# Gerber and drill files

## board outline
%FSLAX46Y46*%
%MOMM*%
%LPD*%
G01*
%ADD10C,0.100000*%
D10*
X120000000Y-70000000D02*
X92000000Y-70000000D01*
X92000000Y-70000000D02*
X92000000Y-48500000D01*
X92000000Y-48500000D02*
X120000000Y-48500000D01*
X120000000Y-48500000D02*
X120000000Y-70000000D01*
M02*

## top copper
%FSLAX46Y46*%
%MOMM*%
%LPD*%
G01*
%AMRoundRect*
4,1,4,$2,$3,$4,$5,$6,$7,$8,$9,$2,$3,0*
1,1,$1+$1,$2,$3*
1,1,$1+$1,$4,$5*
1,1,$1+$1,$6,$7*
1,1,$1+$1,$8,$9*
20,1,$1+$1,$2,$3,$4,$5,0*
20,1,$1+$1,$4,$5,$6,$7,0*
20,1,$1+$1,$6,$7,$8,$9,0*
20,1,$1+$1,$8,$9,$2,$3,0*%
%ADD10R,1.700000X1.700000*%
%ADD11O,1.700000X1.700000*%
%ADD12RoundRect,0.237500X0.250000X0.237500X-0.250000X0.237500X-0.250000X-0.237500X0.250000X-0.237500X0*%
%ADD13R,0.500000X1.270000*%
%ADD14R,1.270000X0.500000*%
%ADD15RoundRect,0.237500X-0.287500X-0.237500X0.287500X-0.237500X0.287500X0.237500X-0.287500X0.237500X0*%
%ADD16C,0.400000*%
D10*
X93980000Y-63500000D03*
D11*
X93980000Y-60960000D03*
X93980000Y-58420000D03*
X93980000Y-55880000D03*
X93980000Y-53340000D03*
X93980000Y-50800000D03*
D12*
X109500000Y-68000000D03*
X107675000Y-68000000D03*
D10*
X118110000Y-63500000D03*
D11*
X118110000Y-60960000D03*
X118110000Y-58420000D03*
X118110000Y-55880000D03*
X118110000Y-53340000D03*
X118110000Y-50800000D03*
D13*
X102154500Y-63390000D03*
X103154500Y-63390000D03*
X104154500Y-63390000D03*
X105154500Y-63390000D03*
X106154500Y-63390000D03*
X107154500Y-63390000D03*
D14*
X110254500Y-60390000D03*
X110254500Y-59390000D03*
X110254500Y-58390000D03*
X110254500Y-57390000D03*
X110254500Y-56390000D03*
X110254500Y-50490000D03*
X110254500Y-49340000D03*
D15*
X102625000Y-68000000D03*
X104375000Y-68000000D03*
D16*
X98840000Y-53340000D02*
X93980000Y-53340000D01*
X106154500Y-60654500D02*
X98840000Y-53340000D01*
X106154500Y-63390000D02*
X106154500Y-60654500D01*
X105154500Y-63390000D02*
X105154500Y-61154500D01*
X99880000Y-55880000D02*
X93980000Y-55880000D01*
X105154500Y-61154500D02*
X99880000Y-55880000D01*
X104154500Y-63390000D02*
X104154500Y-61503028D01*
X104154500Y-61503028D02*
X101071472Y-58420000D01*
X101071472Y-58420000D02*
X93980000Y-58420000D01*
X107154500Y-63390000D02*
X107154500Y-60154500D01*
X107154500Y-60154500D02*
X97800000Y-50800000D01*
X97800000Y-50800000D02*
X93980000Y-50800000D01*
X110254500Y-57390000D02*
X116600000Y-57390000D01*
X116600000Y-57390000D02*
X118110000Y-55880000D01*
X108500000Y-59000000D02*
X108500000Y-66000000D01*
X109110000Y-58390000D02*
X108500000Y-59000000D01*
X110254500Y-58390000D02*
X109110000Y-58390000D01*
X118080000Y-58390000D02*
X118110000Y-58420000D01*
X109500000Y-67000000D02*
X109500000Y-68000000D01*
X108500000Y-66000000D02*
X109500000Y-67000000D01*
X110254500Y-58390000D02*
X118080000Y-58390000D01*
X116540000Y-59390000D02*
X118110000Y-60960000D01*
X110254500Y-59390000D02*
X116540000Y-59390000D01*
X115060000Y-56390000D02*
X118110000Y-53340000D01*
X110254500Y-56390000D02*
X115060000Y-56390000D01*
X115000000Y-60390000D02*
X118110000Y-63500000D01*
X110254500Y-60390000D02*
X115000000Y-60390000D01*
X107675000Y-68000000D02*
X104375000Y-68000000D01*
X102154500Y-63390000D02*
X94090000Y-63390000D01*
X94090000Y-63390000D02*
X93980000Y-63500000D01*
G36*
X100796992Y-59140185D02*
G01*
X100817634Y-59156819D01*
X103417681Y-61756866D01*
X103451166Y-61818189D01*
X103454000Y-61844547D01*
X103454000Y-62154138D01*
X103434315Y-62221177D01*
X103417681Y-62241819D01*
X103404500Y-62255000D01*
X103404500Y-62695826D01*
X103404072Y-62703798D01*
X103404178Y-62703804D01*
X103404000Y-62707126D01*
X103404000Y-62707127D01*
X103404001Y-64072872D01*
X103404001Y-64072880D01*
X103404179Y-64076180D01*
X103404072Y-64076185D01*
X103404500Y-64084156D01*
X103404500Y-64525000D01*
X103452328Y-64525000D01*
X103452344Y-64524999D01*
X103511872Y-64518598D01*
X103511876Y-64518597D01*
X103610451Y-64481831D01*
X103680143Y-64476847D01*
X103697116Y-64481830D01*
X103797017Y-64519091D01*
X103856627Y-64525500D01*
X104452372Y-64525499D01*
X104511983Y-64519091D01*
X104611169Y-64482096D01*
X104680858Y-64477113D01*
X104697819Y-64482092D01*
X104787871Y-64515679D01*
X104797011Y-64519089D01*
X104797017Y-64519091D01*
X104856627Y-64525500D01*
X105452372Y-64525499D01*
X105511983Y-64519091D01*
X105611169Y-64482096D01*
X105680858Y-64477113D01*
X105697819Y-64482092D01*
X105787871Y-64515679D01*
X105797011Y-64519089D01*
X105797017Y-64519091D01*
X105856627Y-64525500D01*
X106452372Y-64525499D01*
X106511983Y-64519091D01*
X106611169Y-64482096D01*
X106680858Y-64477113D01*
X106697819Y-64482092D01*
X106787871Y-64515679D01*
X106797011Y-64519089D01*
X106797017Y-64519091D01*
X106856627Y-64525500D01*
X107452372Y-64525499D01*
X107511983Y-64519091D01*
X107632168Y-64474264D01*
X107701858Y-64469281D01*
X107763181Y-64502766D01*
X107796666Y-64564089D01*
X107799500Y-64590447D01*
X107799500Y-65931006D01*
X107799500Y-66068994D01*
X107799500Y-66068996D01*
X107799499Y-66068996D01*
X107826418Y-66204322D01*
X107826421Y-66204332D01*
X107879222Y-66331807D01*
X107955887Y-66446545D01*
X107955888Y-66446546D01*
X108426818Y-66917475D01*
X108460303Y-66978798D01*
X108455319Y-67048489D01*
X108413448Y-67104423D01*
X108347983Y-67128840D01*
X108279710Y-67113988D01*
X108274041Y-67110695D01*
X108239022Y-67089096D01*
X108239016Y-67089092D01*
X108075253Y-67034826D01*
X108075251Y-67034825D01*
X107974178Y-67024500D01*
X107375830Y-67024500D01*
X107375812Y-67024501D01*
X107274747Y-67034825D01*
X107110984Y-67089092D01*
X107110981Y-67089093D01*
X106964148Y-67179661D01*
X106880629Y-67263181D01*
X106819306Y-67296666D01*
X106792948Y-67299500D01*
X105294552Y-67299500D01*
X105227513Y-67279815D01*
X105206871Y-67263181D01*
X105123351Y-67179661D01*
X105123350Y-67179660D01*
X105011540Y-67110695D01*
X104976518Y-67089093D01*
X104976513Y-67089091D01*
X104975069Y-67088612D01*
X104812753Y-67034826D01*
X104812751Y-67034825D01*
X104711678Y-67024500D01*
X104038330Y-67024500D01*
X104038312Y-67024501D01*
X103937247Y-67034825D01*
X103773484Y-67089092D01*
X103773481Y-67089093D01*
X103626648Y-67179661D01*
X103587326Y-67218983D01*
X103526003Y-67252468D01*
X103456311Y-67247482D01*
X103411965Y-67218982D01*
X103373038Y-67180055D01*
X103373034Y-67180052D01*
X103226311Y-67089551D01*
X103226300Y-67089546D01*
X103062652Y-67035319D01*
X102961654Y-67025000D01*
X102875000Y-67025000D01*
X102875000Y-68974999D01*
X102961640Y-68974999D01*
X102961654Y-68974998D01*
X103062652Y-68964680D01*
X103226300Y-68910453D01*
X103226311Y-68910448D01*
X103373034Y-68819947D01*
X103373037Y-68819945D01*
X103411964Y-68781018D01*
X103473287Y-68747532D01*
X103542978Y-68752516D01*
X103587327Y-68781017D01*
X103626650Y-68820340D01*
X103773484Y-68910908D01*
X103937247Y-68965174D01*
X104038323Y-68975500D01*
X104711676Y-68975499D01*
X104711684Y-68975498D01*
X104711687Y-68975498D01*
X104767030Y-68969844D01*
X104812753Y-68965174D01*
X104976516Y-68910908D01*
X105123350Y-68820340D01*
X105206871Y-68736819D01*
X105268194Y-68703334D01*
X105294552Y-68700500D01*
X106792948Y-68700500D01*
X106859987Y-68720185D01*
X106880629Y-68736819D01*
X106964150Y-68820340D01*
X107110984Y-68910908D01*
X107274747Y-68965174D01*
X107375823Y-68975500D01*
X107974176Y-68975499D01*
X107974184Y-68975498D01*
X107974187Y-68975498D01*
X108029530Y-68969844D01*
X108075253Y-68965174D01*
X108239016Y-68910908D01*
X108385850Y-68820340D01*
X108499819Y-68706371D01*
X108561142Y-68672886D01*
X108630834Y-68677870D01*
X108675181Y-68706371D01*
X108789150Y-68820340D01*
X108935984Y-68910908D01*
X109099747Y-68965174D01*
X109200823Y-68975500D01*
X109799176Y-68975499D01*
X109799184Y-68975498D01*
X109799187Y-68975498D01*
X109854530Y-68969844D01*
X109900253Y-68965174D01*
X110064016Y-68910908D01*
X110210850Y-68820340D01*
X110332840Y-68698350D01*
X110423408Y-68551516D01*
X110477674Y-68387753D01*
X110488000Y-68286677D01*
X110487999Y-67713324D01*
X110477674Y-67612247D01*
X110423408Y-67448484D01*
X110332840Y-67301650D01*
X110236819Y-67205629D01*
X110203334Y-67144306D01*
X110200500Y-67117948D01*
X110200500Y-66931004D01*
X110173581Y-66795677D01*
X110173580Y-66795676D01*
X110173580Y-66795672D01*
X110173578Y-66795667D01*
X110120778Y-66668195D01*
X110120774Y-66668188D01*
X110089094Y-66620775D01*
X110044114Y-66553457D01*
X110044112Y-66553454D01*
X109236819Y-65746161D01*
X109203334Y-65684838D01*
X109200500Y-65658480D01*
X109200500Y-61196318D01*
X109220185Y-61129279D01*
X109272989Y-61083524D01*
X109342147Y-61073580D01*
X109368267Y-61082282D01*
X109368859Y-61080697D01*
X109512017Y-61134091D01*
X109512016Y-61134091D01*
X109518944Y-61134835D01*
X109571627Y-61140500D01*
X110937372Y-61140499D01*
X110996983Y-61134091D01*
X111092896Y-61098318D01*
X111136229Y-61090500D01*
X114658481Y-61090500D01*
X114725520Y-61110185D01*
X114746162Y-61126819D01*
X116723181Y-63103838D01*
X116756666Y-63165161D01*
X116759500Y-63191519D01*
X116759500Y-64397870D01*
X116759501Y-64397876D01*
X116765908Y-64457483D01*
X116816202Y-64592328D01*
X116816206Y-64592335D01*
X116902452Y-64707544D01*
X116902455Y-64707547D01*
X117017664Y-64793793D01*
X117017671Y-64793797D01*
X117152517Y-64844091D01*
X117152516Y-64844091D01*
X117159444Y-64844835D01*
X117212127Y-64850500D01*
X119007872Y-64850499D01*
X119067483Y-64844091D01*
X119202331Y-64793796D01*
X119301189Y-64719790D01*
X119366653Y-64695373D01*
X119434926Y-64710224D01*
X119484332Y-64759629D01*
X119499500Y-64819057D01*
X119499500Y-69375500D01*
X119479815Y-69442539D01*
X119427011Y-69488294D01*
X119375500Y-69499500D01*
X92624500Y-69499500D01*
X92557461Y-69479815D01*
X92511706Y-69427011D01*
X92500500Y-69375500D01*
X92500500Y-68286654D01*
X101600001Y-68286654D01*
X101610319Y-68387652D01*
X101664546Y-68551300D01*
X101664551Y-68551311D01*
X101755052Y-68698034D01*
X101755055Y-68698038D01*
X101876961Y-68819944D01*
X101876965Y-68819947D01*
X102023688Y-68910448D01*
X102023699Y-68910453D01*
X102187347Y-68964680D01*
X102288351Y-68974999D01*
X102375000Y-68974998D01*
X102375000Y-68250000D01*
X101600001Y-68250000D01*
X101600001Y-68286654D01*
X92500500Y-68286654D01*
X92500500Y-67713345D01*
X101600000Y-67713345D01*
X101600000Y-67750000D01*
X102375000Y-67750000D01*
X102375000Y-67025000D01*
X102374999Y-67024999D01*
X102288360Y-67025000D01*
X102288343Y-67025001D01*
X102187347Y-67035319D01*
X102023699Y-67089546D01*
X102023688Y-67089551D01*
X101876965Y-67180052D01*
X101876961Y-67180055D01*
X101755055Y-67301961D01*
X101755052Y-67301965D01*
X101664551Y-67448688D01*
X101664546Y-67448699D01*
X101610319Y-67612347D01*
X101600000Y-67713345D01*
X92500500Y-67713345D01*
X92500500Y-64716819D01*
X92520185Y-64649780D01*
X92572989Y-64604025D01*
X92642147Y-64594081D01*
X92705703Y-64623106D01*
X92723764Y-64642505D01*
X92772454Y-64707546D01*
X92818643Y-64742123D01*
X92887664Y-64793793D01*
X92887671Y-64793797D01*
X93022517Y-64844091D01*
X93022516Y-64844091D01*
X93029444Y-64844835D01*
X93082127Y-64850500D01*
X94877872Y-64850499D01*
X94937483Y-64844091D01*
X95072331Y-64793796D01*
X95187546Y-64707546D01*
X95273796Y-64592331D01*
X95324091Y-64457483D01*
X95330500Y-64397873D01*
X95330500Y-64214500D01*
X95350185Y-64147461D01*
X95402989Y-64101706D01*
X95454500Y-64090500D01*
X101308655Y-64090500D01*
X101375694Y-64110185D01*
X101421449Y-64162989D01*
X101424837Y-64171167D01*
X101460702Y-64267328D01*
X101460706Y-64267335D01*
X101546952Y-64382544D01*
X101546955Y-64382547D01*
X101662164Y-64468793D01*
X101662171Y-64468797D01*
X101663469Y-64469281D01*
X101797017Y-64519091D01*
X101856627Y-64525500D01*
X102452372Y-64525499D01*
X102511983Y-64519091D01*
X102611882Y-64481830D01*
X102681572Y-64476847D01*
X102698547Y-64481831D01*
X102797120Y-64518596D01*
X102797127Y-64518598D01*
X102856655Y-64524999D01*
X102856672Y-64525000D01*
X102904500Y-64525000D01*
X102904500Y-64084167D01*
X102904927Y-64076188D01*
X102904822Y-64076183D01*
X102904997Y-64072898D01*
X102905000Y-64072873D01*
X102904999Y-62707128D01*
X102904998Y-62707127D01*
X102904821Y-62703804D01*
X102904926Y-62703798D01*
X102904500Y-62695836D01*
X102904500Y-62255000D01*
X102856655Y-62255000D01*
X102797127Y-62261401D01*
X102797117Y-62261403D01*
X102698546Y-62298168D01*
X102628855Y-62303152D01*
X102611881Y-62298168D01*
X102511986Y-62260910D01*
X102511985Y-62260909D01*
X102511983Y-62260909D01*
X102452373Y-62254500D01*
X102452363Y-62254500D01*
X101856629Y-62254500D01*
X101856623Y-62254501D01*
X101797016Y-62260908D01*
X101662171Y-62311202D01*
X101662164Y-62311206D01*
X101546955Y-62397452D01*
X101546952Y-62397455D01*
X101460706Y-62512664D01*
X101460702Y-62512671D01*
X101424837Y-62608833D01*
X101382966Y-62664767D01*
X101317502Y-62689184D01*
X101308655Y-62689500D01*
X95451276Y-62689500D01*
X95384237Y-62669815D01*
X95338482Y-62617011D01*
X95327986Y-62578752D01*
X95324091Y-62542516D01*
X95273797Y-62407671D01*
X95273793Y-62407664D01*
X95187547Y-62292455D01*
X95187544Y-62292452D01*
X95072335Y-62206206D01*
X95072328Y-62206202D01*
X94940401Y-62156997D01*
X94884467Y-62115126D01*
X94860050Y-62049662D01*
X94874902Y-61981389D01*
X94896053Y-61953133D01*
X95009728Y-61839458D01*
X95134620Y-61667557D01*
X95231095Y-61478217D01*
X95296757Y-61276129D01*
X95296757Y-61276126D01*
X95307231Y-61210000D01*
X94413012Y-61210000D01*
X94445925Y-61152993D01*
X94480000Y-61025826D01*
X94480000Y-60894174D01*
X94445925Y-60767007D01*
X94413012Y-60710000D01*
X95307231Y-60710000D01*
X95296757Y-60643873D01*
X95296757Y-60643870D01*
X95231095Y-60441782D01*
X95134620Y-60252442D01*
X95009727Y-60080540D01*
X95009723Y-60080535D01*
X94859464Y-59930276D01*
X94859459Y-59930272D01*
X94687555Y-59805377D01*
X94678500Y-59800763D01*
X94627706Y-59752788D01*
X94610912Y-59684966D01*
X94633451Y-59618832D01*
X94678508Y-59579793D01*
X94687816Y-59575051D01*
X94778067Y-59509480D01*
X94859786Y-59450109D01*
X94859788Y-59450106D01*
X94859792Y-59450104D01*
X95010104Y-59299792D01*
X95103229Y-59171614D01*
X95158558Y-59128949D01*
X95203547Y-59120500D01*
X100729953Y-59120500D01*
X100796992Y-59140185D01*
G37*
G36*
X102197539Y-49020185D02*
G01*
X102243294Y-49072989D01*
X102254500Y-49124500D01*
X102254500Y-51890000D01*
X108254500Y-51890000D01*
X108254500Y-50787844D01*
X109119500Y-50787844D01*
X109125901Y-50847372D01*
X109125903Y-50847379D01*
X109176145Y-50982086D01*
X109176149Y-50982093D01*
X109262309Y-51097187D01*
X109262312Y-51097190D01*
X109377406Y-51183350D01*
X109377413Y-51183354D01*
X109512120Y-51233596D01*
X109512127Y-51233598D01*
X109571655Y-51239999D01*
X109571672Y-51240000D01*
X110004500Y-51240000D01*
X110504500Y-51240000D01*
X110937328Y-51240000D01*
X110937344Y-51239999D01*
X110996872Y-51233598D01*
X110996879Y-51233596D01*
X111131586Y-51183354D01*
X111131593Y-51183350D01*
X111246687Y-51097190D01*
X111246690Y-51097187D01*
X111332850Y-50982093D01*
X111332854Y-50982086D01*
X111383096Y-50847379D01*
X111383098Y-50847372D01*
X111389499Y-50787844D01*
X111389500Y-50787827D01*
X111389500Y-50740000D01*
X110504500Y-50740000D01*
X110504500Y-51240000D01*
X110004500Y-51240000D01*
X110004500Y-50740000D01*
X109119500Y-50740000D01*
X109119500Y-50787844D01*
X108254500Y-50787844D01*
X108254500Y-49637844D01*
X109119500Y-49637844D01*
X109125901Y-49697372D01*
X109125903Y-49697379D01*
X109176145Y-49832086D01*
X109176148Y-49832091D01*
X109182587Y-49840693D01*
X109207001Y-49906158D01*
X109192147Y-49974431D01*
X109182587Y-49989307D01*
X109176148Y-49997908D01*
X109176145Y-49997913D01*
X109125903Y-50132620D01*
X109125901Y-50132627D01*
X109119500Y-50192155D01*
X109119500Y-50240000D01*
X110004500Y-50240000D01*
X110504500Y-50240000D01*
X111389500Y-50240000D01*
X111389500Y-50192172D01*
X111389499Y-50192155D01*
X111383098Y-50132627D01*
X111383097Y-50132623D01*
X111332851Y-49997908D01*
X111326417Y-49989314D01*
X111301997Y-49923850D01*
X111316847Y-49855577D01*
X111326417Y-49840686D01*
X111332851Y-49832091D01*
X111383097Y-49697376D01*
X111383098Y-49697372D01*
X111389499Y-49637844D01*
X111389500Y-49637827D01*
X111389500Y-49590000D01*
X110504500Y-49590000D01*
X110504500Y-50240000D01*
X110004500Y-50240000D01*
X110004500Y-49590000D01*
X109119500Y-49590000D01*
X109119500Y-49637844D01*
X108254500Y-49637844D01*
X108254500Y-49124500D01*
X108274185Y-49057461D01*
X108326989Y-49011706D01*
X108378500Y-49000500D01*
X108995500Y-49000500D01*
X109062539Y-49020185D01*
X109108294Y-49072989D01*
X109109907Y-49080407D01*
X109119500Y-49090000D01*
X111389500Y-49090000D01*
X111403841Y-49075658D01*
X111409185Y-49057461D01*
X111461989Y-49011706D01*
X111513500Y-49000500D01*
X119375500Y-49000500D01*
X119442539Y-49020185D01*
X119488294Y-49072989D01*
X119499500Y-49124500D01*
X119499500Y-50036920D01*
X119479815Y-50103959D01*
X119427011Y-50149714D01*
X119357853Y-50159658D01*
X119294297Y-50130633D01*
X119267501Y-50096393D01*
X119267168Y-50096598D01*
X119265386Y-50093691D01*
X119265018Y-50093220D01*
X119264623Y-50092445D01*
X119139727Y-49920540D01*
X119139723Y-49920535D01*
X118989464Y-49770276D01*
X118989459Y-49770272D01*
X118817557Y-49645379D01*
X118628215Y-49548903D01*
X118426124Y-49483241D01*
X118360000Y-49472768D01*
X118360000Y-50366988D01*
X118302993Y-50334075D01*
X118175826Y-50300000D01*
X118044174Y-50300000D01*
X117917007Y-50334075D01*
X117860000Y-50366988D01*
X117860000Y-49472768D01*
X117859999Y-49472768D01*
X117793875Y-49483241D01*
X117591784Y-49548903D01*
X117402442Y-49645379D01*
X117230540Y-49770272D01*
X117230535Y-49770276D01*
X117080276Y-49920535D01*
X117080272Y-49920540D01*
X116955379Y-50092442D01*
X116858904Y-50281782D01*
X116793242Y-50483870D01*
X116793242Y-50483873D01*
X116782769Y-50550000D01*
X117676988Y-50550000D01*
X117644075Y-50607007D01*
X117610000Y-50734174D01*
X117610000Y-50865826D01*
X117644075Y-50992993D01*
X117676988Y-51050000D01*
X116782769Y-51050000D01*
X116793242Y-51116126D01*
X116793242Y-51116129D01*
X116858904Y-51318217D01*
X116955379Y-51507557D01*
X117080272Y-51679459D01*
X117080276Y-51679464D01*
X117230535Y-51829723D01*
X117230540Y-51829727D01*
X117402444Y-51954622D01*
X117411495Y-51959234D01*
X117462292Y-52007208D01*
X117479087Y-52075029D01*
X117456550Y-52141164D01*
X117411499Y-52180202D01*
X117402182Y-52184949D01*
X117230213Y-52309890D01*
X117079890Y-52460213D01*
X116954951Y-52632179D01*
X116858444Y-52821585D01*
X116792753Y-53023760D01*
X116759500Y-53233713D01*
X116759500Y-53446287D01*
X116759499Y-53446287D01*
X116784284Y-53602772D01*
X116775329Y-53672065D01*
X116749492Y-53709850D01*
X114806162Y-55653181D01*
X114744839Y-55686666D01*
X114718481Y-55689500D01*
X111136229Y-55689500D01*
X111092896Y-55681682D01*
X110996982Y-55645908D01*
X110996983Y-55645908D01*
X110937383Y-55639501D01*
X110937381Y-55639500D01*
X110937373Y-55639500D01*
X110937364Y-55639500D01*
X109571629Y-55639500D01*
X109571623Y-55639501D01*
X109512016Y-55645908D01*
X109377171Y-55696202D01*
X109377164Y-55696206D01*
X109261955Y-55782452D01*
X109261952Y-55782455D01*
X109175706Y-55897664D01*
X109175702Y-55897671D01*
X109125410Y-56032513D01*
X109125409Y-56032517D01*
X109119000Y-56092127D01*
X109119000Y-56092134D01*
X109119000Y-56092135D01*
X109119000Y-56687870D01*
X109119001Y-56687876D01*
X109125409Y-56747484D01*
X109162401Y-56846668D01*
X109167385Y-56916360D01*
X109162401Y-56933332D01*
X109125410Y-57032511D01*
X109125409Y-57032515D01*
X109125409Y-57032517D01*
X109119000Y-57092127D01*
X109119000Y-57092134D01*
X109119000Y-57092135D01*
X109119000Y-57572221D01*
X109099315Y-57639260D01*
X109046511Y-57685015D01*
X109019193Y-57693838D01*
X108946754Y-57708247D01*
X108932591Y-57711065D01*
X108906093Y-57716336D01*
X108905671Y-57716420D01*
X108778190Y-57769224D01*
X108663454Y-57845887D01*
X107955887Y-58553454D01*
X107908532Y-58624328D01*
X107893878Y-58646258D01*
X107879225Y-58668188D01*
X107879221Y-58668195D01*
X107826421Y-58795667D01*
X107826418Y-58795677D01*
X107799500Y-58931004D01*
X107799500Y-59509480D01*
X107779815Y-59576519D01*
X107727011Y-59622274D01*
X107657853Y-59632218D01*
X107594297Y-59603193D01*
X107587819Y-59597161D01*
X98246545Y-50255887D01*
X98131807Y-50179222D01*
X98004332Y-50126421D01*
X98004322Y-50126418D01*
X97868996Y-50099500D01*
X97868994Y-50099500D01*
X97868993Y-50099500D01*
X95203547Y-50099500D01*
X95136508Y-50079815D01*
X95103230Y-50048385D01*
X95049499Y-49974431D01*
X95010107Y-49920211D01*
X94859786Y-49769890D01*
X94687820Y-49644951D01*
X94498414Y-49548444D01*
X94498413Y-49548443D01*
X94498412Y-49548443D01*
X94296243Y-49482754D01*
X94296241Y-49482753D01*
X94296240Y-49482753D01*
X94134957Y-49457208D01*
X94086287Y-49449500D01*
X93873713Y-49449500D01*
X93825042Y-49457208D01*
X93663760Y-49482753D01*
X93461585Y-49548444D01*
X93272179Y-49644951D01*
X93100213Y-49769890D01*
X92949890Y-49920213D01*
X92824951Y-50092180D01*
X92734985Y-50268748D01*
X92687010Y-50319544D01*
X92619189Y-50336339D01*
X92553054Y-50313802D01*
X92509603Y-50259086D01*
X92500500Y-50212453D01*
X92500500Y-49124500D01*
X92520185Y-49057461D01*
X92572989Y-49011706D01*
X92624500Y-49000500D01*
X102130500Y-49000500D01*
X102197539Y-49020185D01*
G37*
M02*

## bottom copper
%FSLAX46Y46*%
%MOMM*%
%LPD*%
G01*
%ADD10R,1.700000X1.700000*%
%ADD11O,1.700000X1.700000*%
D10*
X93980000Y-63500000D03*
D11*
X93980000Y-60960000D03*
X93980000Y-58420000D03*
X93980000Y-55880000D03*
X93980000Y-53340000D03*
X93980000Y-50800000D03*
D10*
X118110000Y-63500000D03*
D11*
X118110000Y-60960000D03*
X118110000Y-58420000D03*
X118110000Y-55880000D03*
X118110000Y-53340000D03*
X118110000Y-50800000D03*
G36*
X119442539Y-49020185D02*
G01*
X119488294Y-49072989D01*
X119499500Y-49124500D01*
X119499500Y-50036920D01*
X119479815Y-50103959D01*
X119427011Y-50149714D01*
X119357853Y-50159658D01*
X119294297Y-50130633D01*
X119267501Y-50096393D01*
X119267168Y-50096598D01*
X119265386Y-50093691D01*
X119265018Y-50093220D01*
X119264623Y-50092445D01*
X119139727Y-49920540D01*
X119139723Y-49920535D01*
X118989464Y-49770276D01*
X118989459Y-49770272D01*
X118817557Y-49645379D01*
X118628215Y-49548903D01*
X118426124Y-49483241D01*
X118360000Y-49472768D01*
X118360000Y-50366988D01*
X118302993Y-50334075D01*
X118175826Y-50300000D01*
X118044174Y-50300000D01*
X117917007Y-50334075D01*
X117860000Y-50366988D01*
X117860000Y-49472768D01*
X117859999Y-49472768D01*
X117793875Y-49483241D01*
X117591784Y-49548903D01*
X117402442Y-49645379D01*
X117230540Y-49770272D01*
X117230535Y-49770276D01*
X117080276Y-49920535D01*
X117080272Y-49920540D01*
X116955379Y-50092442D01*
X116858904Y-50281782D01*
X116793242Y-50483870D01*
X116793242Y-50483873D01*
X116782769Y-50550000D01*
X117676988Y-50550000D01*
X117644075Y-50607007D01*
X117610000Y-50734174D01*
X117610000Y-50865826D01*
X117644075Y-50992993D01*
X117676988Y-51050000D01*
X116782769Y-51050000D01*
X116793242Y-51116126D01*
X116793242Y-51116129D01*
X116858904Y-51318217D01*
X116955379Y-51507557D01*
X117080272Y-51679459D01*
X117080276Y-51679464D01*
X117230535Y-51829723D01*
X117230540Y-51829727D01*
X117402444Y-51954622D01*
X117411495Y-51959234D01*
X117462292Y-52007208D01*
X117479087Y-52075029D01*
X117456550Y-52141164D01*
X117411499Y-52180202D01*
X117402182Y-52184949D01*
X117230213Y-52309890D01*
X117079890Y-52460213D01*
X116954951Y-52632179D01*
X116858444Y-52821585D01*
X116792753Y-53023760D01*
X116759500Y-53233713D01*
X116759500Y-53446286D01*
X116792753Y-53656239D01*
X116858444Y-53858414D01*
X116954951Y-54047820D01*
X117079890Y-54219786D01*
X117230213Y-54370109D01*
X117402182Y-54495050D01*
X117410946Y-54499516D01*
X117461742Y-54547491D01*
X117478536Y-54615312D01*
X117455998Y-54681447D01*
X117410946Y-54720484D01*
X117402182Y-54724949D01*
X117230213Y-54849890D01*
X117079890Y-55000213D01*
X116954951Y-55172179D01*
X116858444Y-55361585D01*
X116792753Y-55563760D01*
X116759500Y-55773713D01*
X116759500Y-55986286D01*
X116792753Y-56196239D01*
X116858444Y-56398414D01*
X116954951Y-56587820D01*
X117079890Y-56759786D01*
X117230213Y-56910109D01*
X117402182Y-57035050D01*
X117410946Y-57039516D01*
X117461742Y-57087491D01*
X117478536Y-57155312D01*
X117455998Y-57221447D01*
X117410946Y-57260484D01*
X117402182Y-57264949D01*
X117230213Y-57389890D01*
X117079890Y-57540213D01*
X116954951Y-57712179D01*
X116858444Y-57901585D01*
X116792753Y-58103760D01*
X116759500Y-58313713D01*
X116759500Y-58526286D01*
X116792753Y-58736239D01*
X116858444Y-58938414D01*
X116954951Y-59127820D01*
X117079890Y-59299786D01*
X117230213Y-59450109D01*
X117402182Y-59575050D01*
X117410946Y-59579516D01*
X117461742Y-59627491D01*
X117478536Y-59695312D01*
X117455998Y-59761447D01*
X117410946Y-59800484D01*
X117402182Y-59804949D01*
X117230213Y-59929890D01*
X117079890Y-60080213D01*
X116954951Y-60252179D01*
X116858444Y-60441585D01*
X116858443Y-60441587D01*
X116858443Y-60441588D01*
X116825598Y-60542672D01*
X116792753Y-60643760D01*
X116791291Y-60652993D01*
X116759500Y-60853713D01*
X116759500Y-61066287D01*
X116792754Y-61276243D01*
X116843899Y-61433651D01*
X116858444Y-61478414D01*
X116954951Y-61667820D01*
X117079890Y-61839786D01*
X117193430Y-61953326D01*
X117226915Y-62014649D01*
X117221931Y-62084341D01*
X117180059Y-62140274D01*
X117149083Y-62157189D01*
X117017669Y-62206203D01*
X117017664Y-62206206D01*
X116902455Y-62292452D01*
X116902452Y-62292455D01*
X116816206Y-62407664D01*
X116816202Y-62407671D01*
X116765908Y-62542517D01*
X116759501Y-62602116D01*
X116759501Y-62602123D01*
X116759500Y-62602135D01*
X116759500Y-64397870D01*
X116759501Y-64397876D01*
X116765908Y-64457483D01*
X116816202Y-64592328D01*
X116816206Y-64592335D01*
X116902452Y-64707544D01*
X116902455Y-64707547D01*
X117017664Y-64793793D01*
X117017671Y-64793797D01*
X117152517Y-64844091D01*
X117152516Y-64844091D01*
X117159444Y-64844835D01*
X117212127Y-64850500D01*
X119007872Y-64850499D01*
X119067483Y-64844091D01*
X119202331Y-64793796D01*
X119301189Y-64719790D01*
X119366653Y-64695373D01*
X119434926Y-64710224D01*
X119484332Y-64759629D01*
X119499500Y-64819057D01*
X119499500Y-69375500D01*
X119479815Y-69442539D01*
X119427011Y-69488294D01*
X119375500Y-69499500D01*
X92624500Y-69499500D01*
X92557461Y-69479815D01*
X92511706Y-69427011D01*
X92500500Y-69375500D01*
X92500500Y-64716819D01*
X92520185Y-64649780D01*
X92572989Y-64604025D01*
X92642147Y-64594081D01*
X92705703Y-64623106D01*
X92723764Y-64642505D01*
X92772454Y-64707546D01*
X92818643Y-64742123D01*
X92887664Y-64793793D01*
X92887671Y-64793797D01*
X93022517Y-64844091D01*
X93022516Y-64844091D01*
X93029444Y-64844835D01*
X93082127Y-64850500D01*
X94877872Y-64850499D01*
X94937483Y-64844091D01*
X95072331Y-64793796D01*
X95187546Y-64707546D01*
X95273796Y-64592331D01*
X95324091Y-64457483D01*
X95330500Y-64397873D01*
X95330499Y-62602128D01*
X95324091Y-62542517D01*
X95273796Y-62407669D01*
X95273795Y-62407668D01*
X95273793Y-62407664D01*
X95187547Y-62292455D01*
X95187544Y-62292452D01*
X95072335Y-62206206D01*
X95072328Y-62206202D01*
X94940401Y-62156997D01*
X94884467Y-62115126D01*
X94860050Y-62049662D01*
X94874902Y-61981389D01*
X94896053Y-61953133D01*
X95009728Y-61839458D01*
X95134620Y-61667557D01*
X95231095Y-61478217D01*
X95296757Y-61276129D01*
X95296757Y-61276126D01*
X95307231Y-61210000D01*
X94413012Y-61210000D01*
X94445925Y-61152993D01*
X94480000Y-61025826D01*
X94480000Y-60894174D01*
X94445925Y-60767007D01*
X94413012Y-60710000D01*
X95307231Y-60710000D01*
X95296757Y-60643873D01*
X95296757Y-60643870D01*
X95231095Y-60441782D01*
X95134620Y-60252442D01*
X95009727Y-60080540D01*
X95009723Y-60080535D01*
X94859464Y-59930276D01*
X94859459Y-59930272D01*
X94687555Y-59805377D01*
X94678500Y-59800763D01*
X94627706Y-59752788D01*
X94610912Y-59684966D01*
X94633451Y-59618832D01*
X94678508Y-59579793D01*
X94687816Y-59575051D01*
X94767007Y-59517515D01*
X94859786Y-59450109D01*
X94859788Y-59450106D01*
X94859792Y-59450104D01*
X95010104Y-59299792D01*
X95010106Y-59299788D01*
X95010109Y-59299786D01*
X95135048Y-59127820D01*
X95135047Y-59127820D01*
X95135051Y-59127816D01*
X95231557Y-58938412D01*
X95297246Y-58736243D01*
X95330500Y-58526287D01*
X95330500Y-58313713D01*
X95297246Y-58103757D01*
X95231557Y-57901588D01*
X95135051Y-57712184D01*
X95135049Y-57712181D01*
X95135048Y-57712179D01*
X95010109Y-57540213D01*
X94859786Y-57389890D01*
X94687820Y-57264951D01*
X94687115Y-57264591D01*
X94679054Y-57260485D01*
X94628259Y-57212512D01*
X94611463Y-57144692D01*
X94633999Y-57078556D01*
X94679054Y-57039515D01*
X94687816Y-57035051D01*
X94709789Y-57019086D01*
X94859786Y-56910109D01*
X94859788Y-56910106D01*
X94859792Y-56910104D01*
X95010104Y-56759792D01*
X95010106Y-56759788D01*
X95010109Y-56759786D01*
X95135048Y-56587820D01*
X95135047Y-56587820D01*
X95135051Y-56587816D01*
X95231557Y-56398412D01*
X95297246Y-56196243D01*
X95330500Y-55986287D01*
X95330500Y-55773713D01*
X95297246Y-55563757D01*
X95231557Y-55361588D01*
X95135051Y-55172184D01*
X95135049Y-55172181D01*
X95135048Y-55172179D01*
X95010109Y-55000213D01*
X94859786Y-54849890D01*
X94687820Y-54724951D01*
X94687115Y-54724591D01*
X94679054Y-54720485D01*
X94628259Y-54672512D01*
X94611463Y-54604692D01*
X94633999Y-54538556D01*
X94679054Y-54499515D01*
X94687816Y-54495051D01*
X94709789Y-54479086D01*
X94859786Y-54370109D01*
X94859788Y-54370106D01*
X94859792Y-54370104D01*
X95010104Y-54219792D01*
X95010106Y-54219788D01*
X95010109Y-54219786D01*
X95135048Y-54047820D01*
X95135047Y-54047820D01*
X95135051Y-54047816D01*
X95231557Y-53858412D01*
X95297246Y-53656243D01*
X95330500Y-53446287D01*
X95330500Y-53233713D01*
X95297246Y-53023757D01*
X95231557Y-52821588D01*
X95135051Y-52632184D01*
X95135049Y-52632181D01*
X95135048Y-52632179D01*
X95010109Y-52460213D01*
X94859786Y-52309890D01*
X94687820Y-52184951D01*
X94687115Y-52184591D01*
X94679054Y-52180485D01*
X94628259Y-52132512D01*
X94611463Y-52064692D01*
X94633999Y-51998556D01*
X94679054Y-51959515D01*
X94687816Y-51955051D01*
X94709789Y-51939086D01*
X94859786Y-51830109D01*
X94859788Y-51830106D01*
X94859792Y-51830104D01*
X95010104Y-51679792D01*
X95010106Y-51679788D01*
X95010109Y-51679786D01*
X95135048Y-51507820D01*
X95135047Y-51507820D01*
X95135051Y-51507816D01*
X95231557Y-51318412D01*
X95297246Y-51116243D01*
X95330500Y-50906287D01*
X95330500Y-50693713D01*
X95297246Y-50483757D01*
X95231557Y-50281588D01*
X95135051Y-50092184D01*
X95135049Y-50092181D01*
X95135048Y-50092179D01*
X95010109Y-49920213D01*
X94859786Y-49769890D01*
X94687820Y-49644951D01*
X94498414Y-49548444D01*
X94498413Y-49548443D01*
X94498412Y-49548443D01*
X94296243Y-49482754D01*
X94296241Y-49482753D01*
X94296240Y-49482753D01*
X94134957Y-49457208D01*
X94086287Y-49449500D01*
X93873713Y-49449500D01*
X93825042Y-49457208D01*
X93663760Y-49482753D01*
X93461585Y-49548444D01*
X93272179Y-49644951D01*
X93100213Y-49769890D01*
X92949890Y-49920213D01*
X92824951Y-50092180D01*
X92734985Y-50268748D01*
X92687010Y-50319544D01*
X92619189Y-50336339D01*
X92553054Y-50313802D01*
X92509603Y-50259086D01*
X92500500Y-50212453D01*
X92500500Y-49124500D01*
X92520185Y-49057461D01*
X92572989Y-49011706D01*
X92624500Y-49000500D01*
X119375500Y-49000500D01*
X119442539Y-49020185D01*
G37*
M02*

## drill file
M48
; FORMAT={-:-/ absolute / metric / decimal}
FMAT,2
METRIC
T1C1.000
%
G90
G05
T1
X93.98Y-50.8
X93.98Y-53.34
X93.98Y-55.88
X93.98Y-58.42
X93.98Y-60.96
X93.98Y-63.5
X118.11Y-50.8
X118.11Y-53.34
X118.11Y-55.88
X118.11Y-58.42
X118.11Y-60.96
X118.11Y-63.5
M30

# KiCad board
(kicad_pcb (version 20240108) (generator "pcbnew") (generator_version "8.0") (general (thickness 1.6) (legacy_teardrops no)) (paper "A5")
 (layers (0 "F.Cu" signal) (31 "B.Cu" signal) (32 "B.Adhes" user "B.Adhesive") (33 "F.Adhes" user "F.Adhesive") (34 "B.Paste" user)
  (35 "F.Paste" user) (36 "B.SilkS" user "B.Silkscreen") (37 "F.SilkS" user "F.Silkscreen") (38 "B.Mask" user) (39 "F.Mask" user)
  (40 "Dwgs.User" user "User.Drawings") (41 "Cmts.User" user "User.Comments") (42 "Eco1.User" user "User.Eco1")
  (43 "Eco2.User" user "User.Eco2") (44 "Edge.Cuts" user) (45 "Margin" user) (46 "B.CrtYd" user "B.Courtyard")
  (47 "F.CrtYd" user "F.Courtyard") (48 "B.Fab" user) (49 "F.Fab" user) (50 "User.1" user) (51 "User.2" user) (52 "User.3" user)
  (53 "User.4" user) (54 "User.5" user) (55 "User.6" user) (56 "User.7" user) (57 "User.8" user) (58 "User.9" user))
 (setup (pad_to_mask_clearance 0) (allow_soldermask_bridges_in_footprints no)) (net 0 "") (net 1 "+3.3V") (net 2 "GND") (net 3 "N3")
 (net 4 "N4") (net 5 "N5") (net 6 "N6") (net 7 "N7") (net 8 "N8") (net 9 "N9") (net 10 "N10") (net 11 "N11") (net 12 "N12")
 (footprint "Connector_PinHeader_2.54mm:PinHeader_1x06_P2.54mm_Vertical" (layer "F.Cu") (at 93.98 63.5 180)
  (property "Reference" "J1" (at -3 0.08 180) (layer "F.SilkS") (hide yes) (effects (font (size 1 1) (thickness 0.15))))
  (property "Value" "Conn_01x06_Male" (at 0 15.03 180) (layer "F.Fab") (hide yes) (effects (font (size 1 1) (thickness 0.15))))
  (pad "1" thru_hole rect (at 0 0 180) (size 1.7 1.7) (drill 1) (layers "*.Cu" "*.Mask") (remove_unused_layers no) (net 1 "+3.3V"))
  (pad "2" thru_hole oval (at 0 2.54 180) (size 1.7 1.7) (drill 1) (layers "*.Cu" "*.Mask") (remove_unused_layers no) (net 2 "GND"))
  (pad "3" thru_hole oval (at 0 5.08 180) (size 1.7 1.7) (drill 1) (layers "*.Cu" "*.Mask") (remove_unused_layers no) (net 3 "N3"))
  (pad "4" thru_hole oval (at 0 7.62 180) (size 1.7 1.7) (drill 1) (layers "*.Cu" "*.Mask") (remove_unused_layers no) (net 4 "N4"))
  (pad "5" thru_hole oval (at 0 10.16 180) (size 1.7 1.7) (drill 1) (layers "*.Cu" "*.Mask") (remove_unused_layers no) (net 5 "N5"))
  (pad "6" thru_hole oval (at 0 12.7 180) (size 1.7 1.7) (drill 1) (layers "*.Cu" "*.Mask") (remove_unused_layers no) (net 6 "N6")))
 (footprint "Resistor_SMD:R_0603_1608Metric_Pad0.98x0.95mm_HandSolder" (layer "F.Cu") (at 108.5875 68 180)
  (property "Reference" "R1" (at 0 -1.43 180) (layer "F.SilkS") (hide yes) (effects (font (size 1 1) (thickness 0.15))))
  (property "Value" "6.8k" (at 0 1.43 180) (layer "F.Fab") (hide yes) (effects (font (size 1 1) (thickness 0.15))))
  (pad "1" smd roundrect (at -0.9125 0 180) (size 0.975 0.95) (layers "F.Cu" "F.Paste" "F.Mask") (roundrect_rratio 0.25) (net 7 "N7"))
  (pad "2" smd roundrect (at 0.9125 0 180) (size 0.975 0.95) (layers "F.Cu" "F.Paste" "F.Mask") (roundrect_rratio 0.25) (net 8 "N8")))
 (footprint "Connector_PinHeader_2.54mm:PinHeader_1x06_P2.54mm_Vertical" (layer "F.Cu") (at 118.11 63.5 180)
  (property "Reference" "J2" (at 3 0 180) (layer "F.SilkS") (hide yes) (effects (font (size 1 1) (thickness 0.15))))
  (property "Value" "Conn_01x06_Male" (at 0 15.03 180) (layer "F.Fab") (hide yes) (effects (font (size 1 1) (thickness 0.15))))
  (pad "1" thru_hole rect (at 0 0 180) (size 1.7 1.7) (drill 1) (layers "*.Cu" "*.Mask") (remove_unused_layers no) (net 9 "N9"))
  (pad "2" thru_hole oval (at 0 2.54 180) (size 1.7 1.7) (drill 1) (layers "*.Cu" "*.Mask") (remove_unused_layers no) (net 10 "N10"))
  (pad "3" thru_hole oval (at 0 5.08 180) (size 1.7 1.7) (drill 1) (layers "*.Cu" "*.Mask") (remove_unused_layers no) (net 7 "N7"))
  (pad "4" thru_hole oval (at 0 7.62 180) (size 1.7 1.7) (drill 1) (layers "*.Cu" "*.Mask") (remove_unused_layers no) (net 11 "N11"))
  (pad "5" thru_hole oval (at 0 10.16 180) (size 1.7 1.7) (drill 1) (layers "*.Cu" "*.Mask") (remove_unused_layers no) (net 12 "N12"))
  (pad "6" thru_hole oval (at 0 12.7 180) (size 1.7 1.7) (drill 1) (layers "*.Cu" "*.Mask") (remove_unused_layers no) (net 2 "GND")))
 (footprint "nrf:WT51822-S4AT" (layer "F.Cu") (at 110.2545 63.39 90)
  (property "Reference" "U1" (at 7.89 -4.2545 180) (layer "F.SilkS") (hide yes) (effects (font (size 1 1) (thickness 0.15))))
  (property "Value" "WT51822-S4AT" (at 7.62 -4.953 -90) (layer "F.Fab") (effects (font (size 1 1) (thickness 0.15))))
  (pad "1" smd rect (at 0 -8.1 90) (size 1.27 0.5) (layers "F.Cu" "F.Paste" "F.Mask") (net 1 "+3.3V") (solder_mask_margin 0.102))
  (pad "2" smd rect (at 0 -7.1 90) (size 1.27 0.5) (layers "F.Cu" "F.Paste" "F.Mask") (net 2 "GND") (solder_mask_margin 0.102))
  (pad "3" smd rect (at 0 -6.1 90) (size 1.27 0.5) (layers "F.Cu" "F.Paste" "F.Mask") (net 3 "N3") (solder_mask_margin 0.102))
  (pad "4" smd rect (at 0 -5.1 90) (size 1.27 0.5) (layers "F.Cu" "F.Paste" "F.Mask") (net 4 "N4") (solder_mask_margin 0.102))
  (pad "5" smd rect (at 0 -4.1 90) (size 1.27 0.5) (layers "F.Cu" "F.Paste" "F.Mask") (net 5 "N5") (solder_mask_margin 0.102))
  (pad "6" smd rect (at 0 -3.1 90) (size 1.27 0.5) (layers "F.Cu" "F.Paste" "F.Mask") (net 6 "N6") (solder_mask_margin 0.102))
  (pad "7" smd rect (at 3 0) (size 1.27 0.5) (layers "F.Cu" "F.Paste" "F.Mask") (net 9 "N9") (solder_mask_margin 0.102))
  (pad "8" smd rect (at 4 0) (size 1.27 0.5) (layers "F.Cu" "F.Paste" "F.Mask") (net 10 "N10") (solder_mask_margin 0.102))
  (pad "9" smd rect (at 5 0) (size 1.27 0.5) (layers "F.Cu" "F.Paste" "F.Mask") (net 7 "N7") (solder_mask_margin 0.102))
  (pad "10" smd rect (at 6 0) (size 1.27 0.5) (layers "F.Cu" "F.Paste" "F.Mask") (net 11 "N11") (solder_mask_margin 0.102))
  (pad "11" smd rect (at 7 0) (size 1.27 0.5) (layers "F.Cu" "F.Paste" "F.Mask") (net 12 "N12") (solder_mask_margin 0.102))
  (pad "12" smd rect (at 12.9 0) (size 1.27 0.5) (layers "F.Cu" "F.Paste" "F.Mask") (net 2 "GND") (solder_mask_margin 0.102))
  (pad "13" smd rect (at 14.05 0) (size 1.27 0.5) (layers "F.Cu" "F.Paste" "F.Mask") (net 2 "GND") (solder_mask_margin 0.102))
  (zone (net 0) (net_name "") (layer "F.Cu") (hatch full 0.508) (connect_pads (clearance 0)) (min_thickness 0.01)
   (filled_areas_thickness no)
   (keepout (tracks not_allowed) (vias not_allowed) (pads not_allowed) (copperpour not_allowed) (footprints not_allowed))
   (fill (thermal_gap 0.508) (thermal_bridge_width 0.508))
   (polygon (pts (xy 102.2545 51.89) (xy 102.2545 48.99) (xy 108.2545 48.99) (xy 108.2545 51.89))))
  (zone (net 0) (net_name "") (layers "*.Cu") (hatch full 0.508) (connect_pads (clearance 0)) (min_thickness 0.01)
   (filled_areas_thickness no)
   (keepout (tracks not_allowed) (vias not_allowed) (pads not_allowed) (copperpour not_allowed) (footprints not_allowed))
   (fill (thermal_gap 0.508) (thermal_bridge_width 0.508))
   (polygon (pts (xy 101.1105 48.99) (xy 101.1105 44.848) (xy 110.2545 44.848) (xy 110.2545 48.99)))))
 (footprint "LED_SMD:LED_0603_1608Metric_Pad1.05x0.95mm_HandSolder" (layer "F.Cu") (at 103.5 68)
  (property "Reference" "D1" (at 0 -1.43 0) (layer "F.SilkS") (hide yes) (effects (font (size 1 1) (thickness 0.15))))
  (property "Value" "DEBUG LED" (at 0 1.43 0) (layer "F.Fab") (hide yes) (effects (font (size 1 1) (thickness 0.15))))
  (pad "1" smd roundrect (at -0.875 0) (size 1.05 0.95) (layers "F.Cu" "F.Paste" "F.Mask") (roundrect_rratio 0.25) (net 2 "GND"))
  (pad "2" smd roundrect (at 0.875 0) (size 1.05 0.95) (layers "F.Cu" "F.Paste" "F.Mask") (roundrect_rratio 0.25) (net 8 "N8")))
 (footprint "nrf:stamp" (layer "B.Cu") (at 105.5 56.5 180)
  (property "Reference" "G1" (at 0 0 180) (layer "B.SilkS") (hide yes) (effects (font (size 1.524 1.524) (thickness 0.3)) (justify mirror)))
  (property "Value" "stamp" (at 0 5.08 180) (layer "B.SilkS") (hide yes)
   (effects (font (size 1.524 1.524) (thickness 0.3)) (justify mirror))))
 (gr_line (start 120 70) (end 92 70) (stroke (width 0.1) (type default)) (layer "Edge.Cuts"))
 (gr_line (start 92 70) (end 92 48.5) (stroke (width 0.1) (type default)) (layer "Edge.Cuts"))
 (gr_line (start 92 48.5) (end 120 48.5) (stroke (width 0.1) (type default)) (layer "Edge.Cuts"))
 (gr_line (start 120 48.5) (end 120 70) (stroke (width 0.1) (type default)) (layer "Edge.Cuts"))
 (segment (start 98.84 53.34) (end 93.98 53.34) (width 0.4) (layer "F.Cu") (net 5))
 (segment (start 106.1545 60.6545) (end 98.84 53.34) (width 0.4) (layer "F.Cu") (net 5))
 (segment (start 106.1545 63.39) (end 106.1545 60.6545) (width 0.4) (layer "F.Cu") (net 5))
 (segment (start 105.1545 63.39) (end 105.1545 61.1545) (width 0.4) (layer "F.Cu") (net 4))
 (segment (start 99.88 55.88) (end 93.98 55.88) (width 0.4) (layer "F.Cu") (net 4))
 (segment (start 105.1545 61.1545) (end 99.88 55.88) (width 0.4) (layer "F.Cu") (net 4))
 (segment (start 104.1545 63.39) (end 104.1545 61.503028) (width 0.4) (layer "F.Cu") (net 3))
 (segment (start 104.1545 61.503028) (end 101.071472 58.42) (width 0.4) (layer "F.Cu") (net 3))
 (segment (start 101.071472 58.42) (end 93.98 58.42) (width 0.4) (layer "F.Cu") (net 3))
 (segment (start 107.1545 63.39) (end 107.1545 60.1545) (width 0.4) (layer "F.Cu") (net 6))
 (segment (start 107.1545 60.1545) (end 97.8 50.8) (width 0.4) (layer "F.Cu") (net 6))
 (segment (start 97.8 50.8) (end 93.98 50.8) (width 0.4) (layer "F.Cu") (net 6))
 (segment (start 110.2545 57.39) (end 116.6 57.39) (width 0.4) (layer "F.Cu") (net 11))
 (segment (start 116.6 57.39) (end 118.11 55.88) (width 0.4) (layer "F.Cu") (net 11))
 (segment (start 108.5 59) (end 108.5 66) (width 0.4) (layer "F.Cu") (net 7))
 (segment (start 109.11 58.39) (end 108.5 59) (width 0.4) (layer "F.Cu") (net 7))
 (segment (start 110.2545 58.39) (end 109.11 58.39) (width 0.4) (layer "F.Cu") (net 7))
 (segment (start 118.08 58.39) (end 118.11 58.42) (width 0.4) (layer "F.Cu") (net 7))
 (segment (start 109.5 67) (end 109.5 68) (width 0.4) (layer "F.Cu") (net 7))
 (segment (start 108.5 66) (end 109.5 67) (width 0.4) (layer "F.Cu") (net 7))
 (segment (start 110.2545 58.39) (end 118.08 58.39) (width 0.4) (layer "F.Cu") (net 7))
 (segment (start 116.54 59.39) (end 118.11 60.96) (width 0.4) (layer "F.Cu") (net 10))
 (segment (start 110.2545 59.39) (end 116.54 59.39) (width 0.4) (layer "F.Cu") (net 10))
 (segment (start 115.06 56.39) (end 118.11 53.34) (width 0.4) (layer "F.Cu") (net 12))
 (segment (start 110.2545 56.39) (end 115.06 56.39) (width 0.4) (layer "F.Cu") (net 12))
 (segment (start 115 60.39) (end 118.11 63.5) (width 0.4) (layer "F.Cu") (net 9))
 (segment (start 110.2545 60.39) (end 115 60.39) (width 0.4) (layer "F.Cu") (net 9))
 (segment (start 107.675 68) (end 104.375 68) (width 0.4) (layer "F.Cu") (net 8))
 (segment (start 102.1545 63.39) (end 94.09 63.39) (width 0.4) (layer "F.Cu") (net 1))
 (segment (start 94.09 63.39) (end 93.98 63.5) (width 0.4) (layer "F.Cu") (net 1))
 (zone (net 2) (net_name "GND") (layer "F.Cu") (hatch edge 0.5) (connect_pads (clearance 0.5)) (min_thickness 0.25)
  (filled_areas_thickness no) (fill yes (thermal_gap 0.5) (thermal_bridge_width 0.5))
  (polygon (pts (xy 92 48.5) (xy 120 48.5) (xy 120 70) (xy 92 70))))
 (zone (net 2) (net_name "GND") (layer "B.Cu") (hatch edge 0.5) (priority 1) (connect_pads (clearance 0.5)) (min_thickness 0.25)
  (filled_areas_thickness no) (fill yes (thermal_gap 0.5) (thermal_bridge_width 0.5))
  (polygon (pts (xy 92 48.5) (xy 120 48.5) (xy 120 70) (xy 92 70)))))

